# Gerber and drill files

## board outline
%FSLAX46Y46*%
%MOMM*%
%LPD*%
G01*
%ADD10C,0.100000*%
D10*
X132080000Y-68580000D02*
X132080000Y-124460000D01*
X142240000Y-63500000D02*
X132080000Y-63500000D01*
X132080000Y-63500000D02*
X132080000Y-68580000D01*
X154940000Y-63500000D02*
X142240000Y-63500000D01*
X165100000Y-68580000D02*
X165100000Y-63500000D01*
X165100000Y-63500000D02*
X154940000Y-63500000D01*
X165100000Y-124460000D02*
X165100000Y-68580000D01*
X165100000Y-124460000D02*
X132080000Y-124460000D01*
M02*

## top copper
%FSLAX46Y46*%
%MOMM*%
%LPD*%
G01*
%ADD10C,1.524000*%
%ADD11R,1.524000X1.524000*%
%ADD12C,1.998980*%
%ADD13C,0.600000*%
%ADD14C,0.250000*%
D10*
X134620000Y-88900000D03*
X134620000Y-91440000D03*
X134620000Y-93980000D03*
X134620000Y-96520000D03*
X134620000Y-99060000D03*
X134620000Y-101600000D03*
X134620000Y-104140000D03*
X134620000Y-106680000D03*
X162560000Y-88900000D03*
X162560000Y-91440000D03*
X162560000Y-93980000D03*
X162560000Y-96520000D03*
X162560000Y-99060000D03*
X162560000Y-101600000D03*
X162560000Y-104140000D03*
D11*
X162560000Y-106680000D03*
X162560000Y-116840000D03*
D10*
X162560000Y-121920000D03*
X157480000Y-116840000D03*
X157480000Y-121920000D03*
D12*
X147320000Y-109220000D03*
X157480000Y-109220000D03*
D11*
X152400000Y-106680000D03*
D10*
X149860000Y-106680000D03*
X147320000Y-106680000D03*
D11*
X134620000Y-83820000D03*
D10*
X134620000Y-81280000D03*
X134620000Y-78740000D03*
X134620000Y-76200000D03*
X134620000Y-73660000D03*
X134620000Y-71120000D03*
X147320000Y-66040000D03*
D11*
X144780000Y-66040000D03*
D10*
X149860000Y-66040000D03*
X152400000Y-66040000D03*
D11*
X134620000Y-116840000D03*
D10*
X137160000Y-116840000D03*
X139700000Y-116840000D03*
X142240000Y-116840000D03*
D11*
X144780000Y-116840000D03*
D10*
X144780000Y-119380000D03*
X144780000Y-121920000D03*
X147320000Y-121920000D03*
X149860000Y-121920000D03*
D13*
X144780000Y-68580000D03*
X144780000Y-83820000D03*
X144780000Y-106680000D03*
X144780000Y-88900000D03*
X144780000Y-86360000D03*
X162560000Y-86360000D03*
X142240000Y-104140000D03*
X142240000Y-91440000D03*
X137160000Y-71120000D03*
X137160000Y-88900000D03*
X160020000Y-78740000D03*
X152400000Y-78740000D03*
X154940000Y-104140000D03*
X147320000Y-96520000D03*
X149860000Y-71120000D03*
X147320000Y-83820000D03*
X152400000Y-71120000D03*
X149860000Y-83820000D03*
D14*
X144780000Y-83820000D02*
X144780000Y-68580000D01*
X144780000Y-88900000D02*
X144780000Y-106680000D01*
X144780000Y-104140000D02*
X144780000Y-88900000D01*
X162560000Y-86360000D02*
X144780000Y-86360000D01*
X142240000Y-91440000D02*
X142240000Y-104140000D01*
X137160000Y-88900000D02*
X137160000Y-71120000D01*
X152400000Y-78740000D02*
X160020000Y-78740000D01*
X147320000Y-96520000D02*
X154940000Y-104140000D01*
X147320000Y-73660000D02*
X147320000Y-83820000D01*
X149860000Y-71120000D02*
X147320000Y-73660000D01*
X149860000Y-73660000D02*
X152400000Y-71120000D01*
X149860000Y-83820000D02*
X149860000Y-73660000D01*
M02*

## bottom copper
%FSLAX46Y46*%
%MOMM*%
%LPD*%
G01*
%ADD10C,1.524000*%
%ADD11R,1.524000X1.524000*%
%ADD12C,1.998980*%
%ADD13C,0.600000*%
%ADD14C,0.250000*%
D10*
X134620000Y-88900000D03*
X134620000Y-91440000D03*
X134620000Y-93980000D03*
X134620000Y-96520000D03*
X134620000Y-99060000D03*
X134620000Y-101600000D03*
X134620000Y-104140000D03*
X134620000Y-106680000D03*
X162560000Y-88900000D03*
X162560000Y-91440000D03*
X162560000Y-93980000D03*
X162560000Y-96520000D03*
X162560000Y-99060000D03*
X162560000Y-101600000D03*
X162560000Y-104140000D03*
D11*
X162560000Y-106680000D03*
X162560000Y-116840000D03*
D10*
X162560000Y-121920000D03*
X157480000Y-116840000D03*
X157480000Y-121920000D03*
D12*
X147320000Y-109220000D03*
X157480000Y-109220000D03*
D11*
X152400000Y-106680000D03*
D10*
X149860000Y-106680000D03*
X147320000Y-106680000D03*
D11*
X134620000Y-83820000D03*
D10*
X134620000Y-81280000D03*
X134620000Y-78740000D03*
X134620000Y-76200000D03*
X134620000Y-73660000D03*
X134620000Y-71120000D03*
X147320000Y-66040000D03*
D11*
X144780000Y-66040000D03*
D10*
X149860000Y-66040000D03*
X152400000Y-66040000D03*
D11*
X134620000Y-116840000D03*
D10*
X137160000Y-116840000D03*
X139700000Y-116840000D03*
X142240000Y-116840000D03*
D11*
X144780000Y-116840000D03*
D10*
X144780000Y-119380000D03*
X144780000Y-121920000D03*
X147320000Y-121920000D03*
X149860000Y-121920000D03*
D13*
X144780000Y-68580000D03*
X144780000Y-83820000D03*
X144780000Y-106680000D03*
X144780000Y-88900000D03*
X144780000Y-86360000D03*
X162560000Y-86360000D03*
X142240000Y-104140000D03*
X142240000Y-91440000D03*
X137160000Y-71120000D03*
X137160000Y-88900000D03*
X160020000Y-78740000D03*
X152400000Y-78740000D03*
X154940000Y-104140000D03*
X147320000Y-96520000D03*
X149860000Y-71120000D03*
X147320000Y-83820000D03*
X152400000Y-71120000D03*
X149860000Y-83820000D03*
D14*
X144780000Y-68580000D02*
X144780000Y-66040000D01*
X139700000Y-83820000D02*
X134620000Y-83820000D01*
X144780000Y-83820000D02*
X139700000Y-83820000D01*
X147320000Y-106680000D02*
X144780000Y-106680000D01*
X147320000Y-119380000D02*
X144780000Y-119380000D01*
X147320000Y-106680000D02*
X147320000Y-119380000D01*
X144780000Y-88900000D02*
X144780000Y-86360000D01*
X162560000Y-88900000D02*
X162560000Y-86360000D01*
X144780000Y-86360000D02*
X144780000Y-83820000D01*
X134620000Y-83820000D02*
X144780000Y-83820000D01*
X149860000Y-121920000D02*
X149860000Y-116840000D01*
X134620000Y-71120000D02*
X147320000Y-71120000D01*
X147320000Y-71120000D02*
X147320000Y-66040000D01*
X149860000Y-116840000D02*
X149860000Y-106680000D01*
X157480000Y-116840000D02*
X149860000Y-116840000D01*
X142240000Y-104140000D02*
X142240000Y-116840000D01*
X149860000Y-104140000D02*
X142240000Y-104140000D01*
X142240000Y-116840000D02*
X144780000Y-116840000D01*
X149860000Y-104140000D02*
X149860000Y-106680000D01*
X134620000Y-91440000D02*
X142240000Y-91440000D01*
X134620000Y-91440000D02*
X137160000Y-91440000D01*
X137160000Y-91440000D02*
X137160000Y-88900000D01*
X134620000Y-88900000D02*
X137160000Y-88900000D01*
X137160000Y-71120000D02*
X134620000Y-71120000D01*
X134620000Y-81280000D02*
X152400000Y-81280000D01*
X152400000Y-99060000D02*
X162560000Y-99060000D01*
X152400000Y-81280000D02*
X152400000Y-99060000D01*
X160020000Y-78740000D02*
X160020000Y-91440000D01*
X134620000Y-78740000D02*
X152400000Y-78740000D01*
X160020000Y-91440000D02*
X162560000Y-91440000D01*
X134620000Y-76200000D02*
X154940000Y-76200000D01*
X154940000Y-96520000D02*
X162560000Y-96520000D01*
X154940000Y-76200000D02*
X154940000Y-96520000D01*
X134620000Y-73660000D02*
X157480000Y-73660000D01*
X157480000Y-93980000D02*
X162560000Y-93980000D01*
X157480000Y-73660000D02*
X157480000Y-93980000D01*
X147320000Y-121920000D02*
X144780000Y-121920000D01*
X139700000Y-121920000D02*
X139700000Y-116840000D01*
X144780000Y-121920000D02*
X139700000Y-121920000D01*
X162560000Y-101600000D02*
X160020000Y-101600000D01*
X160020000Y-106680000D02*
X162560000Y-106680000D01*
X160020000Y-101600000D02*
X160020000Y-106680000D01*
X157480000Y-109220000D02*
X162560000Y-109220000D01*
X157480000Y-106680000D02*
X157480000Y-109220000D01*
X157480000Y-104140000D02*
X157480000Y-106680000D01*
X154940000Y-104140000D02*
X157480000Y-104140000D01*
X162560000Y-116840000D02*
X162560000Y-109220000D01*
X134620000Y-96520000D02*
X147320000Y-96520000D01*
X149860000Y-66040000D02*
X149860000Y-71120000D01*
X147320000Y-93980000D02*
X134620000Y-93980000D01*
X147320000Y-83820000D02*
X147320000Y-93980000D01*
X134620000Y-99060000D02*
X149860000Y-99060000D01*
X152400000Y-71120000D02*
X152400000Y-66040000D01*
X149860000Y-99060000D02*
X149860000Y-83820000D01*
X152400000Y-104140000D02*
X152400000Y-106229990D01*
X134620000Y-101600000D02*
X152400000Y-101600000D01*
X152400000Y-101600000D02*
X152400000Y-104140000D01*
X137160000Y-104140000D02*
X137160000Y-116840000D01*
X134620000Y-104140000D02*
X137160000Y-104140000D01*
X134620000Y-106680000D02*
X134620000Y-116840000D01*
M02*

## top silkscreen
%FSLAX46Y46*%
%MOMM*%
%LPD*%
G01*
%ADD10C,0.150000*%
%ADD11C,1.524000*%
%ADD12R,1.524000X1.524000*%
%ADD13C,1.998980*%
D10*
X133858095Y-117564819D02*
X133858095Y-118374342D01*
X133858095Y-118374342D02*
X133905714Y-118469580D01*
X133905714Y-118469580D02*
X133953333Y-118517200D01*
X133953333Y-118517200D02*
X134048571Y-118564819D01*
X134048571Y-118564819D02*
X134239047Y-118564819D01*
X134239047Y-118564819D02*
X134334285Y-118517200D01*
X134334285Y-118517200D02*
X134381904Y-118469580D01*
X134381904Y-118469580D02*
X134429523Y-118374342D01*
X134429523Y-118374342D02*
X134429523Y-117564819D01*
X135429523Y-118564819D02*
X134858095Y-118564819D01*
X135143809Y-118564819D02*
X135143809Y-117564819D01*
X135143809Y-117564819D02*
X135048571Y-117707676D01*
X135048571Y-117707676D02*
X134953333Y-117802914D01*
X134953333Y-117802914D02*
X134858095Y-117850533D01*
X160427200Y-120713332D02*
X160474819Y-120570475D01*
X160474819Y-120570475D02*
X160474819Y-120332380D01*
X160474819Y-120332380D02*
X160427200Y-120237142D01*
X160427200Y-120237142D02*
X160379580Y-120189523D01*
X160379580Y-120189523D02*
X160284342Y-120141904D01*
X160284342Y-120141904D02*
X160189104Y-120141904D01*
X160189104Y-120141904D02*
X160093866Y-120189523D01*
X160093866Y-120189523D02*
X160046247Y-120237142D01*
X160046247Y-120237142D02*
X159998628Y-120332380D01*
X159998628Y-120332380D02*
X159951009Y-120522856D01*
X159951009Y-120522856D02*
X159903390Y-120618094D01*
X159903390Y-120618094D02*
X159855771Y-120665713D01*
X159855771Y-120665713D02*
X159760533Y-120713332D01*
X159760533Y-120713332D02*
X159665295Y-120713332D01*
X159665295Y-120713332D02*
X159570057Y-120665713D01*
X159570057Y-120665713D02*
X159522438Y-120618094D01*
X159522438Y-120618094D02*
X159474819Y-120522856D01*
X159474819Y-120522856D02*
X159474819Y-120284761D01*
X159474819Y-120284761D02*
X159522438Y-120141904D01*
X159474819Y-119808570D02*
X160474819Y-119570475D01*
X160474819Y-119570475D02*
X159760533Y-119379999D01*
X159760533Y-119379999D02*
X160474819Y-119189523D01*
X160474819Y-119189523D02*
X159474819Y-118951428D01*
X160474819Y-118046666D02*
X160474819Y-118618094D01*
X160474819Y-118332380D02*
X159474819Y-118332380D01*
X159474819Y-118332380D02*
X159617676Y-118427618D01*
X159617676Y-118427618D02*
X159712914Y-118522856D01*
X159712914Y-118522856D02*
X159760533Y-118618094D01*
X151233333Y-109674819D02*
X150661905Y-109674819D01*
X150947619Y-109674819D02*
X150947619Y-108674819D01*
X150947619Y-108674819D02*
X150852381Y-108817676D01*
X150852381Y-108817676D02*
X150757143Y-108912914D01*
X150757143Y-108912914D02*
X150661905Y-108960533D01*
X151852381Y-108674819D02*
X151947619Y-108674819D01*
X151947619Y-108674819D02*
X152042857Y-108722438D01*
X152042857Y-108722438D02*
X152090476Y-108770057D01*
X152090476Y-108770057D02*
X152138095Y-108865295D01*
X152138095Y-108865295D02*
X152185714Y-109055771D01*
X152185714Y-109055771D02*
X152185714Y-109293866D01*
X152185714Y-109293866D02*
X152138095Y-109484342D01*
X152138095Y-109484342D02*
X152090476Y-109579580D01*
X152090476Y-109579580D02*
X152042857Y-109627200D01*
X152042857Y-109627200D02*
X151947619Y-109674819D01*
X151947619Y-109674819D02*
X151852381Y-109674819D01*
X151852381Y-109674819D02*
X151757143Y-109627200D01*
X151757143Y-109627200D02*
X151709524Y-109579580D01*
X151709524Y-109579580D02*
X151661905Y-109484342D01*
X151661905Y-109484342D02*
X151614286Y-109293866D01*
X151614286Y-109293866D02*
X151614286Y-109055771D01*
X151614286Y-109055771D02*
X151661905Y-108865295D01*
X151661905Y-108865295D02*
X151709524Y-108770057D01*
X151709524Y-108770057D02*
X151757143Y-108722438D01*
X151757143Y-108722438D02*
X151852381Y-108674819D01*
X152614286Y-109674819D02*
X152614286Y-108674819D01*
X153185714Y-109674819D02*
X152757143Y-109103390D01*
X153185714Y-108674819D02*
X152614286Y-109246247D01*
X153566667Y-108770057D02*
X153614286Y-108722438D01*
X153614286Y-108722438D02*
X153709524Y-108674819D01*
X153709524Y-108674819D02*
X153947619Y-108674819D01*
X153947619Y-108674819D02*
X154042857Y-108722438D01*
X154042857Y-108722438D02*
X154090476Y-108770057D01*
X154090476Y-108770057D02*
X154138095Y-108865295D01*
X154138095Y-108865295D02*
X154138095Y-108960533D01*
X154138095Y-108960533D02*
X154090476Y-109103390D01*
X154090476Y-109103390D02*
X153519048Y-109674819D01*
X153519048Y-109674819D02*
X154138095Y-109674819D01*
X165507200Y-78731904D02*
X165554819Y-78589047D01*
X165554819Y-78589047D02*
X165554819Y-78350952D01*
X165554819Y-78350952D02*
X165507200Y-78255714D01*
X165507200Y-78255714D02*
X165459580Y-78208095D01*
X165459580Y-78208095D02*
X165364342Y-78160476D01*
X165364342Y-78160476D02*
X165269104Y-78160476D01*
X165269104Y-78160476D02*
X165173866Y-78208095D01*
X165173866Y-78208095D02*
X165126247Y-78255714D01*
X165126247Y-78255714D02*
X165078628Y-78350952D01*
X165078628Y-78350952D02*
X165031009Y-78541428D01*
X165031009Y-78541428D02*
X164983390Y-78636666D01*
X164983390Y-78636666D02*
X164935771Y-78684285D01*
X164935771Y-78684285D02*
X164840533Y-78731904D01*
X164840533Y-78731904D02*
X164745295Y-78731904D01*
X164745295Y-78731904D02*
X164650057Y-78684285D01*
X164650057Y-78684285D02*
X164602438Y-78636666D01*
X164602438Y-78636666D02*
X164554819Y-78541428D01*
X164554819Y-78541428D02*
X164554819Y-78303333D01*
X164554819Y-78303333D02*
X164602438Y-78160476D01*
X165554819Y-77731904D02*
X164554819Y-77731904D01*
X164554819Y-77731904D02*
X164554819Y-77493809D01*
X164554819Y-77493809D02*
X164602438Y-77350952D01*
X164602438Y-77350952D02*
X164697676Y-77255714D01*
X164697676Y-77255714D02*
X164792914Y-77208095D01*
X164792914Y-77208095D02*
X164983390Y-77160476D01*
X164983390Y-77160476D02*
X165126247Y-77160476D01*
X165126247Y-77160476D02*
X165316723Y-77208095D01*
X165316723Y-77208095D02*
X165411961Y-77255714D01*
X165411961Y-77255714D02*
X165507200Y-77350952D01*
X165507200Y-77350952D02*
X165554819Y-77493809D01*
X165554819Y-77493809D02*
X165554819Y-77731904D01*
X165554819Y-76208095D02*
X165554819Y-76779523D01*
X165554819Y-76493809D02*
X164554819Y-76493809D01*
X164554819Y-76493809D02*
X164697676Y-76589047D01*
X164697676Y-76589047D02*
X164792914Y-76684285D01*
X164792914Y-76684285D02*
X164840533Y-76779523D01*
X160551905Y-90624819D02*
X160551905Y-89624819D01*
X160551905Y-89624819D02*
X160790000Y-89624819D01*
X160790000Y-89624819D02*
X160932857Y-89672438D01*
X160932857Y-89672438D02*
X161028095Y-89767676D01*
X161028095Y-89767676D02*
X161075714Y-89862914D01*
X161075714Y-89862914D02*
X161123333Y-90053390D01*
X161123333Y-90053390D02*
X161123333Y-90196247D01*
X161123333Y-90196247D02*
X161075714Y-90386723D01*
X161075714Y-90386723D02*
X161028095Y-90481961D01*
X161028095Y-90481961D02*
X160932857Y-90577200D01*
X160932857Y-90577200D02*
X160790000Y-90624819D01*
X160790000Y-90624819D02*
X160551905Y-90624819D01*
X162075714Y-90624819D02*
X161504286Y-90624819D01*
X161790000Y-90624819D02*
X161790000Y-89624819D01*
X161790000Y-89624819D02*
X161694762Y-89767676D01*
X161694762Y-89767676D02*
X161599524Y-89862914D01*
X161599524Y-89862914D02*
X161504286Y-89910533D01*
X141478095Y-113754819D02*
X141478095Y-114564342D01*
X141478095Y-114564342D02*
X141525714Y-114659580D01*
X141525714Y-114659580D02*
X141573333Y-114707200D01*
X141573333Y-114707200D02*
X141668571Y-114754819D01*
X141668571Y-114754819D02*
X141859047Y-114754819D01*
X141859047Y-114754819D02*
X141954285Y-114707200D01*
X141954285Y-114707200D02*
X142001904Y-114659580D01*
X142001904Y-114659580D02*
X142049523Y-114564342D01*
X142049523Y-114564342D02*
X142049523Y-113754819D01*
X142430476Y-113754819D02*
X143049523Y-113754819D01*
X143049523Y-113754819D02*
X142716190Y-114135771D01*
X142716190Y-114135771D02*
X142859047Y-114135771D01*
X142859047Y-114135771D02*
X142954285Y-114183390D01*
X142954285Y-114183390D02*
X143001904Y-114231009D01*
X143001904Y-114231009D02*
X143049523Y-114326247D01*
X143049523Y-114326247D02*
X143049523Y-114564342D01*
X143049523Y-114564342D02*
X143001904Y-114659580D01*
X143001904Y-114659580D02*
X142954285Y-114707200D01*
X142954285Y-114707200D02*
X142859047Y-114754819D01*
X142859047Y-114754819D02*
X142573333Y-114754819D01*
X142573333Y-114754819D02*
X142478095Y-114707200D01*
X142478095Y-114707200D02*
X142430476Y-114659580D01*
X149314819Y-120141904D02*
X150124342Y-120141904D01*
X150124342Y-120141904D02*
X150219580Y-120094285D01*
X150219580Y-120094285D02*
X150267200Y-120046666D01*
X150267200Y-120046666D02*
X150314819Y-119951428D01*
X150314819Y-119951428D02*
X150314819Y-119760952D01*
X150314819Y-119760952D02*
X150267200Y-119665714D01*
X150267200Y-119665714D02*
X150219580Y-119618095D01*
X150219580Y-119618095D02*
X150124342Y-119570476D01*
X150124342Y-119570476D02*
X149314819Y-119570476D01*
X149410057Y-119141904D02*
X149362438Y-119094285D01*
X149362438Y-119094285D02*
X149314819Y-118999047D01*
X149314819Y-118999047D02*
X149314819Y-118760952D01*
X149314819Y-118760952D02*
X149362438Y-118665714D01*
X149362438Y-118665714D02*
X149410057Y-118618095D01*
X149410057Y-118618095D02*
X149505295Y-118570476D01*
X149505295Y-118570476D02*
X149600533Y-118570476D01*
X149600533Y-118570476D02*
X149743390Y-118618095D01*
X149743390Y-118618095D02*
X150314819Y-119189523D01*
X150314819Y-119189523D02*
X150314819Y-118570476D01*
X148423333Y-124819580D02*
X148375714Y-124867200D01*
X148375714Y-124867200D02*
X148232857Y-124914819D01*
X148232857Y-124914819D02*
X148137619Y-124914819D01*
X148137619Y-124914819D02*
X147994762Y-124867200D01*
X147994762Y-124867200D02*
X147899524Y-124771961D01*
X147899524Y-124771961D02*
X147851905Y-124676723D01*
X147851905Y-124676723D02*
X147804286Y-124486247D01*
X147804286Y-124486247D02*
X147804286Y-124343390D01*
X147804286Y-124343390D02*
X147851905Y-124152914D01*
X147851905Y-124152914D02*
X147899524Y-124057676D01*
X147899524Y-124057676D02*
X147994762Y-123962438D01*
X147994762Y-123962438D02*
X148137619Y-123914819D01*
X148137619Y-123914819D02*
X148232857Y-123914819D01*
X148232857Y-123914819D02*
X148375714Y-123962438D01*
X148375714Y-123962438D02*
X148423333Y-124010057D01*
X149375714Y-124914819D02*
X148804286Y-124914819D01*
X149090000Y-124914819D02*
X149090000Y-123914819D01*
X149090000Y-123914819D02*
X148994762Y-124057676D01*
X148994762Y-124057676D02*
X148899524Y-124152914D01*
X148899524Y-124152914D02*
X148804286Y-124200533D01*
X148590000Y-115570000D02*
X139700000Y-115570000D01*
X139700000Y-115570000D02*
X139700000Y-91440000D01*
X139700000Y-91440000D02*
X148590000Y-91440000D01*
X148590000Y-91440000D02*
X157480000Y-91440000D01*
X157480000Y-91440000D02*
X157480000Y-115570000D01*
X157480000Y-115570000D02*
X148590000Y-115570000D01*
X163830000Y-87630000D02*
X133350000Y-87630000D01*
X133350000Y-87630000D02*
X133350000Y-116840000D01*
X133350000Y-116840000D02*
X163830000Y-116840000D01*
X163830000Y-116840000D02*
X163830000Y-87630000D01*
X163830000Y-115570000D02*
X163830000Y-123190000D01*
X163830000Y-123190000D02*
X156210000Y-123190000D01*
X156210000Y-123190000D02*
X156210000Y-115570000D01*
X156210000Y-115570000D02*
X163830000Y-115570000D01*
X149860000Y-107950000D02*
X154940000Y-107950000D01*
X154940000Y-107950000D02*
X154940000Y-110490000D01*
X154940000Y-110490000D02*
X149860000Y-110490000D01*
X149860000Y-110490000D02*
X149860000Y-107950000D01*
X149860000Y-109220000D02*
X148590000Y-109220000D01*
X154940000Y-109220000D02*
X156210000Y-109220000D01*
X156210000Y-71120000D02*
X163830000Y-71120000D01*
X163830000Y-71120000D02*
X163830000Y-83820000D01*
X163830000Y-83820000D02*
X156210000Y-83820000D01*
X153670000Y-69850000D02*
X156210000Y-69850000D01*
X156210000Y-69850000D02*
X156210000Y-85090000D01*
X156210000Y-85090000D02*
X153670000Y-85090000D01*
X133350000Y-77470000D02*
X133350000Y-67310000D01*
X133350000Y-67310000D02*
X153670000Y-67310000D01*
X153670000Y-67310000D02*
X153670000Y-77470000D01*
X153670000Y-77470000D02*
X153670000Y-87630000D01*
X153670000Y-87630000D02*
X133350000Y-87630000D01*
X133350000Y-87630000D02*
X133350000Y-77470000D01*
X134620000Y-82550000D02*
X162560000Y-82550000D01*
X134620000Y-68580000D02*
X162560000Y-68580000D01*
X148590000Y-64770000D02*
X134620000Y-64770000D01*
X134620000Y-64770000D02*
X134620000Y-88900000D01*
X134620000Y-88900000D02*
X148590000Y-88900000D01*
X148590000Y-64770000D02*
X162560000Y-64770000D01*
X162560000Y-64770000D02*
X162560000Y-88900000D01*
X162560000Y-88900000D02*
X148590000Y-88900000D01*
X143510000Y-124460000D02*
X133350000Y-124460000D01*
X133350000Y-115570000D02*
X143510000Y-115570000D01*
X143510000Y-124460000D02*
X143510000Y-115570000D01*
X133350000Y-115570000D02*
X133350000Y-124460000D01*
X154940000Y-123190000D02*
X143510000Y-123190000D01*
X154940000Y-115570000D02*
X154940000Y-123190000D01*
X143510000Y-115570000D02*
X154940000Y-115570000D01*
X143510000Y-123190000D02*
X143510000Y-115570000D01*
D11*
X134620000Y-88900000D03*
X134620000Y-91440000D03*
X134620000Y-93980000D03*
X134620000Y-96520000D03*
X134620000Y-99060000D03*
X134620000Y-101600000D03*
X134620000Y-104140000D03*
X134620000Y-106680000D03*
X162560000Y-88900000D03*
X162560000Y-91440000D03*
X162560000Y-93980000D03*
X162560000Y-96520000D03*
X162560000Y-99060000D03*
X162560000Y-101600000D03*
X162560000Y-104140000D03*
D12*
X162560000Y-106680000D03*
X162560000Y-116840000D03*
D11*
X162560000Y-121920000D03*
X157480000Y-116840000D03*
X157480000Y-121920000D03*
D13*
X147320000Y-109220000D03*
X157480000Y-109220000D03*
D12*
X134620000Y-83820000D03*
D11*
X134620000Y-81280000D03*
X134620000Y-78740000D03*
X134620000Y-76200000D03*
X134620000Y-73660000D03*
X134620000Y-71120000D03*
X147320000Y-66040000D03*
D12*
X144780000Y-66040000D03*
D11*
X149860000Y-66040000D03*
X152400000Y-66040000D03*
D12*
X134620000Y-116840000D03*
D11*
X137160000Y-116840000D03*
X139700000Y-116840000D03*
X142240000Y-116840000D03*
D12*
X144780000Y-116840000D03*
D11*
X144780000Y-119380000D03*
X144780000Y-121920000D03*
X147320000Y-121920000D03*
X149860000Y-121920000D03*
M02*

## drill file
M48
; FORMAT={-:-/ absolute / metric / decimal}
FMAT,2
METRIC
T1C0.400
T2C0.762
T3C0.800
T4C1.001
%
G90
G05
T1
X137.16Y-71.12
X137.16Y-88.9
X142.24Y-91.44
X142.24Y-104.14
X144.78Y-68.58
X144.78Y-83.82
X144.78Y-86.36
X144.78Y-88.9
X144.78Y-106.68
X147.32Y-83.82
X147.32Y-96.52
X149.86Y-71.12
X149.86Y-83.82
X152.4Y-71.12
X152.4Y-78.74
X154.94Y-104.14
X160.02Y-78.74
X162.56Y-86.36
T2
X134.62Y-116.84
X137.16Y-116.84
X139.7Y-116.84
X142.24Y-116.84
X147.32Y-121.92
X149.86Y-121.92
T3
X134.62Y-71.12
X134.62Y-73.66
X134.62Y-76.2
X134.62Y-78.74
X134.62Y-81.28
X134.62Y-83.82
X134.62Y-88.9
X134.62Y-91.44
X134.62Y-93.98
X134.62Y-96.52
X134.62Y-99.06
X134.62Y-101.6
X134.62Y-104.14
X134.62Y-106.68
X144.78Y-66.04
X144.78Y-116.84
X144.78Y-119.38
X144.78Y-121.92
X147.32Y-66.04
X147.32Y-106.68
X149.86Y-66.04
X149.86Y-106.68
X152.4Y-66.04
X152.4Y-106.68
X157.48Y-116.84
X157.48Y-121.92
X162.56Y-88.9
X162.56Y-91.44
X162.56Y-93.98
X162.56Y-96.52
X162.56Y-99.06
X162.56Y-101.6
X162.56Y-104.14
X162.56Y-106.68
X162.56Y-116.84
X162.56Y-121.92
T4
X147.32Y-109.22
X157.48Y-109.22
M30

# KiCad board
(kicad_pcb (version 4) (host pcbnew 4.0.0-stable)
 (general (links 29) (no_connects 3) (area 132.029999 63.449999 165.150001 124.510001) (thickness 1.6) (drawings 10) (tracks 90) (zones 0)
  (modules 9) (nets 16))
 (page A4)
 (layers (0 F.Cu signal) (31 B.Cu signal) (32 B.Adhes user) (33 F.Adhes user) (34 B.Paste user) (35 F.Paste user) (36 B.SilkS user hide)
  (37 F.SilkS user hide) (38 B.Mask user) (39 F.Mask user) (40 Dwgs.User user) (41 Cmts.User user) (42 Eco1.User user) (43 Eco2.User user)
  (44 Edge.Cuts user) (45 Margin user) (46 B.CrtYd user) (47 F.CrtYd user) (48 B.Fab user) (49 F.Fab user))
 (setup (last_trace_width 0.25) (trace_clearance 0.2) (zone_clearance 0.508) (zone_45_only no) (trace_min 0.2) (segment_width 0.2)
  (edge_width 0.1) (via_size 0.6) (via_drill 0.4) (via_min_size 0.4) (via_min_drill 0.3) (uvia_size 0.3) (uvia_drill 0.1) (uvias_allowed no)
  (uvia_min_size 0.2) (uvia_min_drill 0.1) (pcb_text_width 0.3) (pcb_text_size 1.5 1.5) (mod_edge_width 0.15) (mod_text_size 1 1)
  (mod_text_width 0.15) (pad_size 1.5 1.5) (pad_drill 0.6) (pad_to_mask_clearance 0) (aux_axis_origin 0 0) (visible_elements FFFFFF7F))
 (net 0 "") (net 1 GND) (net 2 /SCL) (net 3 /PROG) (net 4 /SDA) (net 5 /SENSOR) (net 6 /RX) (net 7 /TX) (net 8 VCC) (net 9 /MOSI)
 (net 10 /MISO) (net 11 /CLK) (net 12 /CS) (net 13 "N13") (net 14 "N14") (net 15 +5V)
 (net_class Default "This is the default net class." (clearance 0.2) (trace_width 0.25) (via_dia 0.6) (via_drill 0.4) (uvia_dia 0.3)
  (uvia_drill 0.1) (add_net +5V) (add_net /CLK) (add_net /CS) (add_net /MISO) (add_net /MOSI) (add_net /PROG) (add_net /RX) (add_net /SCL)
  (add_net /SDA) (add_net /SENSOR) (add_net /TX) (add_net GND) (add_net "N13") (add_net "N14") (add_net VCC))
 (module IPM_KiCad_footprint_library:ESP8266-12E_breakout (layer F.Cu) (at 162.56 106.68 180)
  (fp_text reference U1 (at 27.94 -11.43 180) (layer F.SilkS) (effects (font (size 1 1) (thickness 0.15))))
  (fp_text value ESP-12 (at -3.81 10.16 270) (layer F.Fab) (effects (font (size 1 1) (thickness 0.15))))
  (fp_line (start 13.97 -8.89) (end 22.86 -8.89) (layer F.SilkS) (width 0.15))
  (fp_line (start 22.86 -8.89) (end 22.86 15.24) (layer F.SilkS) (width 0.15))
  (fp_line (start 22.86 15.24) (end 13.97 15.24) (layer F.SilkS) (width 0.15))
  (fp_line (start 13.97 15.24) (end 5.08 15.24) (layer F.SilkS) (width 0.15))
  (fp_line (start 5.08 15.24) (end 5.08 -8.89) (layer F.SilkS) (width 0.15))
  (fp_line (start 5.08 -8.89) (end 13.97 -8.89) (layer F.SilkS) (width 0.15))
  (fp_line (start -1.27 19.05) (end 29.21 19.05) (layer F.SilkS) (width 0.15))
  (fp_line (start 29.21 19.05) (end 29.21 -10.16) (layer F.SilkS) (width 0.15))
  (fp_line (start 29.21 -10.16) (end -1.27 -10.16) (layer F.SilkS) (width 0.15))
  (fp_line (start -1.27 -10.16) (end -1.27 19.05) (layer F.SilkS) (width 0.15))
  (pad 9 thru_hole circle (at 27.94 17.78 180) (size 1.524 1.524) (drill 0.8) (layers *.Cu *.Mask F.SilkS) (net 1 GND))
  (pad 10 thru_hole circle (at 27.94 15.24 180) (size 1.524 1.524) (drill 0.8) (layers *.Cu *.Mask F.SilkS) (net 1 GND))
  (pad 11 thru_hole circle (at 27.94 12.7 180) (size 1.524 1.524) (drill 0.8) (layers *.Cu *.Mask F.SilkS) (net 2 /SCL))
  (pad 12 thru_hole circle (at 27.94 10.16 180) (size 1.524 1.524) (drill 0.8) (layers *.Cu *.Mask F.SilkS) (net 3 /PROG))
  (pad 13 thru_hole circle (at 27.94 7.62 180) (size 1.524 1.524) (drill 0.8) (layers *.Cu *.Mask F.SilkS) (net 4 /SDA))
  (pad 14 thru_hole circle (at 27.94 5.08 180) (size 1.524 1.524) (drill 0.8) (layers *.Cu *.Mask F.SilkS) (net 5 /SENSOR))
  (pad 15 thru_hole circle (at 27.94 2.54 180) (size 1.524 1.524) (drill 0.8) (layers *.Cu *.Mask F.SilkS) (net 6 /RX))
  (pad 16 thru_hole circle (at 27.94 0 180) (size 1.524 1.524) (drill 0.8) (layers *.Cu *.Mask F.SilkS) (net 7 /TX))
  (pad 8 thru_hole circle (at 0 17.78 180) (size 1.524 1.524) (drill 0.8) (layers *.Cu *.Mask F.SilkS) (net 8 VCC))
  (pad 7 thru_hole circle (at 0 15.24 180) (size 1.524 1.524) (drill 0.8) (layers *.Cu *.Mask F.SilkS) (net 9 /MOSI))
  (pad 6 thru_hole circle (at 0 12.7 180) (size 1.524 1.524) (drill 0.8) (layers *.Cu *.Mask F.SilkS) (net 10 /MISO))
  (pad 5 thru_hole circle (at 0 10.16 180) (size 1.524 1.524) (drill 0.8) (layers *.Cu *.Mask F.SilkS) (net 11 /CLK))
  (pad 4 thru_hole circle (at 0 7.62 180) (size 1.524 1.524) (drill 0.8) (layers *.Cu *.Mask F.SilkS) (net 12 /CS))
  (pad 3 thru_hole circle (at 0 5.08 180) (size 1.524 1.524) (drill 0.8) (layers *.Cu *.Mask F.SilkS) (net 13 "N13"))
  (pad 2 thru_hole circle (at 0 2.54 180) (size 1.524 1.524) (drill 0.8) (layers *.Cu *.Mask F.SilkS) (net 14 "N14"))
  (pad 1 thru_hole rect (at 0 0 180) (size 1.524 1.524) (drill 0.8) (layers *.Cu *.Mask F.SilkS) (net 13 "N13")))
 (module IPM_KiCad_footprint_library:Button (layer F.Cu) (at 162.56 116.84 270)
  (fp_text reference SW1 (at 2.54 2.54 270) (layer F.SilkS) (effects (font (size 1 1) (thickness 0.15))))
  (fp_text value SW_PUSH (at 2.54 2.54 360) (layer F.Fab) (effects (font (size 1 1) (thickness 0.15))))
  (fp_line (start -1.27 -1.27) (end 6.35 -1.27) (layer F.SilkS) (width 0.15))
  (fp_line (start 6.35 -1.27) (end 6.35 6.35) (layer F.SilkS) (width 0.15))
  (fp_line (start 6.35 6.35) (end -1.27 6.35) (layer F.SilkS) (width 0.15))
  (fp_line (start -1.27 6.35) (end -1.27 -1.27) (layer F.SilkS) (width 0.15))
  (pad 1 thru_hole rect (at 0 0 270) (size 1.524 1.524) (drill 0.8) (layers *.Cu *.Mask F.SilkS) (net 3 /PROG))
  (pad 1 thru_hole circle (at 5.08 0 270) (size 1.524 1.524) (drill 0.8) (layers *.Cu *.Mask F.SilkS) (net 3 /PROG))
  (pad 2 thru_hole circle (at 0 5.08 270) (size 1.524 1.524) (drill 0.8) (layers *.Cu *.Mask F.SilkS) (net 1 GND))
  (pad 2 thru_hole circle (at 5.08 5.08 270) (size 1.524 1.524) (drill 0.8) (layers *.Cu *.Mask F.SilkS) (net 1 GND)))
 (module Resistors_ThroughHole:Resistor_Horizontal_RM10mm (layer F.Cu) (at 152.4 109.22)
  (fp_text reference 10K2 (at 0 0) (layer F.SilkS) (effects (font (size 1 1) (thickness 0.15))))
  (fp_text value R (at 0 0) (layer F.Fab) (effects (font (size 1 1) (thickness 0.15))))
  (fp_line (start -2.54 -1.27) (end 2.54 -1.27) (layer F.SilkS) (width 0.15))
  (fp_line (start 2.54 -1.27) (end 2.54 1.27) (layer F.SilkS) (width 0.15))
  (fp_line (start 2.54 1.27) (end -2.54 1.27) (layer F.SilkS) (width 0.15))
  (fp_line (start -2.54 1.27) (end -2.54 -1.27) (layer F.SilkS) (width 0.15))
  (fp_line (start -2.54 0) (end -3.81 0) (layer F.SilkS) (width 0.15))
  (fp_line (start 2.54 0) (end 3.81 0) (layer F.SilkS) (width 0.15))
  (pad 1 thru_hole circle (at -5.08 0) (size 1.99898 1.99898) (drill 1.00076) (layers *.Cu *.SilkS *.Mask) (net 8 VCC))
  (pad 2 thru_hole circle (at 5.08 0) (size 1.99898 1.99898) (drill 1.00076) (layers *.Cu *.SilkS *.Mask) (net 3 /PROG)))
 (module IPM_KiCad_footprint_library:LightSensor (layer B.Cu) (at 152.4 106.68 180)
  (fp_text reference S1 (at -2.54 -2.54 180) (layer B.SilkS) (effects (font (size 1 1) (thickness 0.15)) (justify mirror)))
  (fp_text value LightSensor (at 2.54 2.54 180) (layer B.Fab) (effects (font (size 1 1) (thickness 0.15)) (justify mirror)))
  (pad 1 thru_hole rect (at 0 0 180) (size 1.524 1.524) (drill 0.8) (layers *.Cu *.Mask B.SilkS) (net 5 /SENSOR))
  (pad 2 thru_hole circle (at 2.54 0 180) (size 1.524 1.524) (drill 0.8) (layers *.Cu *.Mask B.SilkS) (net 1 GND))
  (pad 3 thru_hole circle (at 5.08 0 180) (size 1.524 1.524) (drill 0.8) (layers *.Cu *.Mask B.SilkS) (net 8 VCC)))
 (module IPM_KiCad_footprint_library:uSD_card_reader (layer F.Cu) (at 134.62 83.82 90)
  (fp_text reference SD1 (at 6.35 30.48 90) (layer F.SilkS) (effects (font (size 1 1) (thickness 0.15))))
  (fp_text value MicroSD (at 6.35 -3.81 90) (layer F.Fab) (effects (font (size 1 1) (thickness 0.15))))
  (fp_line (start 12.7 21.59) (end 12.7 29.21) (layer F.SilkS) (width 0.15))
  (fp_line (start 12.7 29.21) (end 0 29.21) (layer F.SilkS) (width 0.15))
  (fp_line (start 0 29.21) (end 0 21.59) (layer F.SilkS) (width 0.15))
  (fp_line (start 13.97 19.05) (end 13.97 21.59) (layer F.SilkS) (width 0.15))
  (fp_line (start 13.97 21.59) (end -1.27 21.59) (layer F.SilkS) (width 0.15))
  (fp_line (start -1.27 21.59) (end -1.27 19.05) (layer F.SilkS) (width 0.15))
  (fp_line (start 6.35 -1.27) (end 16.51 -1.27) (layer F.SilkS) (width 0.15))
  (fp_line (start 16.51 -1.27) (end 16.51 19.05) (layer F.SilkS) (width 0.15))
  (fp_line (start 16.51 19.05) (end 6.35 19.05) (layer F.SilkS) (width 0.15))
  (fp_line (start 6.35 19.05) (end -3.81 19.05) (layer F.SilkS) (width 0.15))
  (fp_line (start -3.81 19.05) (end -3.81 -1.27) (layer F.SilkS) (width 0.15))
  (fp_line (start -3.81 -1.27) (end 6.35 -1.27) (layer F.SilkS) (width 0.15))
  (pad 1 thru_hole rect (at 0 0 90) (size 1.524 1.524) (drill 0.8) (layers *.Cu *.Mask F.SilkS) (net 8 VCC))
  (pad 2 thru_hole circle (at 2.54 0 90) (size 1.524 1.524) (drill 0.8) (layers *.Cu *.Mask F.SilkS) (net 12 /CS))
  (pad 3 thru_hole circle (at 5.08 0 90) (size 1.524 1.524) (drill 0.8) (layers *.Cu *.Mask F.SilkS) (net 9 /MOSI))
  (pad 4 thru_hole circle (at 7.62 0 90) (size 1.524 1.524) (drill 0.8) (layers *.Cu *.Mask F.SilkS) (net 11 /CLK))
  (pad 5 thru_hole circle (at 10.16 0 90) (size 1.524 1.524) (drill 0.8) (layers *.Cu *.Mask F.SilkS) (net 10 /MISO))
  (pad 6 thru_hole circle (at 12.7 0 90) (size 1.524 1.524) (drill 0.8) (layers *.Cu *.Mask F.SilkS) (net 1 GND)))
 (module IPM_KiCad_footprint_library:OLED (layer F.Cu) (at 144.78 66.04)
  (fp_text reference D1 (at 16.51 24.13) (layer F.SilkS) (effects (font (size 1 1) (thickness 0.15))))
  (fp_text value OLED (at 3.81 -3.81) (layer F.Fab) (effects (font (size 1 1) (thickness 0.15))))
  (fp_line (start -10.16 16.51) (end 17.78 16.51) (layer F.SilkS) (width 0.15))
  (fp_line (start -10.16 2.54) (end 17.78 2.54) (layer F.SilkS) (width 0.15))
  (fp_line (start 3.81 -1.27) (end -10.16 -1.27) (layer F.SilkS) (width 0.15))
  (fp_line (start -10.16 -1.27) (end -10.16 22.86) (layer F.SilkS) (width 0.15))
  (fp_line (start -10.16 22.86) (end 3.81 22.86) (layer F.SilkS) (width 0.15))
  (fp_line (start 3.81 -1.27) (end 17.78 -1.27) (layer F.SilkS) (width 0.15))
  (fp_line (start 17.78 -1.27) (end 17.78 22.86) (layer F.SilkS) (width 0.15))
  (fp_line (start 17.78 22.86) (end 3.81 22.86) (layer F.SilkS) (width 0.15))
  (pad 2 thru_hole circle (at 2.54 0) (size 1.524 1.524) (drill 0.8) (layers *.Cu *.Mask F.SilkS) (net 1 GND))
  (pad 1 thru_hole rect (at 0 0) (size 1.524 1.524) (drill 0.8) (layers *.Cu *.Mask F.SilkS) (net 8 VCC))
  (pad 3 thru_hole circle (at 5.08 0) (size 1.524 1.524) (drill 0.8) (layers *.Cu *.Mask F.SilkS) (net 2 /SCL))
  (pad 4 thru_hole circle (at 7.62 0) (size 1.524 1.524) (drill 0.8) (layers *.Cu *.Mask F.SilkS) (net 4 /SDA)))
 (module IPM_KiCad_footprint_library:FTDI (layer F.Cu) (at 134.62 116.84)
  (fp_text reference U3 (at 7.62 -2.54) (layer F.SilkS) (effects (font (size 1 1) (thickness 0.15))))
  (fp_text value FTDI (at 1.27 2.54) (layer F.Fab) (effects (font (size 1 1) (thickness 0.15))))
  (fp_line (start 8.89 7.62) (end -1.27 7.62) (layer F.SilkS) (width 0.15))
  (fp_line (start -1.27 -1.27) (end 8.89 -1.27) (layer F.SilkS) (width 0.15))
  (fp_line (start 8.89 7.62) (end 8.89 -1.27) (layer F.SilkS) (width 0.15))
  (fp_line (start -1.27 -1.27) (end -1.27 7.62) (layer F.SilkS) (width 0.15))
  (pad 1 thru_hole rect (at 0 0) (size 1.524 1.524) (drill 0.762) (layers *.Cu *.Mask F.SilkS) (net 7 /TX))
  (pad 2 thru_hole circle (at 2.54 0) (size 1.524 1.524) (drill 0.762) (layers *.Cu *.Mask F.SilkS) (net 6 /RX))
  (pad 3 thru_hole circle (at 5.08 0) (size 1.524 1.524) (drill 0.762) (layers *.Cu *.Mask F.SilkS) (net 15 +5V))
  (pad 4 thru_hole circle (at 7.62 0) (size 1.524 1.524) (drill 0.762) (layers *.Cu *.Mask F.SilkS) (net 1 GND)))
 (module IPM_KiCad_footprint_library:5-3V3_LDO (layer F.Cu) (at 144.78 116.84 90)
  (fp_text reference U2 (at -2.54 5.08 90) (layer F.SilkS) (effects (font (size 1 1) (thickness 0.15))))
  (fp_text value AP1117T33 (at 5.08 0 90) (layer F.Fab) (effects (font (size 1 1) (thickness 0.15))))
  (fp_line (start -6.35 10.16) (end -6.35 -1.27) (layer F.SilkS) (width 0.15))
  (fp_line (start 1.27 10.16) (end -6.35 10.16) (layer F.SilkS) (width 0.15))
  (fp_line (start 1.27 -1.27) (end 1.27 10.16) (layer F.SilkS) (width 0.15))
  (fp_line (start -6.35 -1.27) (end 1.27 -1.27) (layer F.SilkS) (width 0.15))
  (pad 1 thru_hole rect (at 0 0 90) (size 1.524 1.524) (drill 0.8) (layers *.Cu *.Mask F.SilkS) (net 1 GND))
  (pad 2 thru_hole circle (at -2.54 0 90) (size 1.524 1.524) (drill 0.8) (layers *.Cu *.Mask F.SilkS) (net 8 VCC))
  (pad 3 thru_hole circle (at -5.08 0 90) (size 1.524 1.524) (drill 0.8) (layers *.Cu *.Mask F.SilkS) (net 15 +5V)))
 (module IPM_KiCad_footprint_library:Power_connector (layer F.Cu) (at 148.59 121.92)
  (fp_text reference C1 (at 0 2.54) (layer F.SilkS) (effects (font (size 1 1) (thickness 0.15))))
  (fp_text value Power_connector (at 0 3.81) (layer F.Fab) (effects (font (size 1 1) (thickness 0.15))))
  (pad 1 thru_hole circle (at -1.27 0) (size 1.524 1.524) (drill 0.762) (layers *.Cu *.Mask F.SilkS) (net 15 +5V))
  (pad 2 thru_hole circle (at 1.27 0) (size 1.524 1.524) (drill 0.762) (layers *.Cu *.Mask F.SilkS) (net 1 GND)))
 (gr_line (start 132.08 68.58) (end 132.08 124.46) (angle 90) (layer Edge.Cuts) (width 0.1))
 (gr_line (start 142.24 63.5) (end 132.08 63.5) (angle 90) (layer Edge.Cuts) (width 0.1))
 (gr_line (start 132.08 63.5) (end 132.08 68.58) (angle 90) (layer Edge.Cuts) (width 0.1))
 (gr_line (start 154.94 63.5) (end 142.24 63.5) (angle 90) (layer Edge.Cuts) (width 0.1))
 (gr_line (start 165.1 68.58) (end 165.1 63.5) (angle 90) (layer Edge.Cuts) (width 0.1))
 (gr_line (start 165.1 63.5) (end 154.94 63.5) (angle 90) (layer Edge.Cuts) (width 0.1))
 (gr_line (start 165.1 124.46) (end 165.1 68.58) (angle 90) (layer Edge.Cuts) (width 0.1))
 (gr_line (start 165.1 124.46) (end 132.08 124.46) (angle 90) (layer Edge.Cuts) (width 0.1))
 (segment (start 144.78 68.58) (end 144.78 66.04) (width 0.25) (layer B.Cu) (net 8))
 (via (at 144.78 68.58) (size 0.6) (drill 0.4) (layers F.Cu B.Cu) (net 8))
 (segment (start 144.78 83.82) (end 144.78 68.58) (width 0.25) (layer F.Cu) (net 8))
 (segment (start 139.7 83.82) (end 134.62 83.82) (width 0.25) (layer B.Cu) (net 8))
 (segment (start 144.78 83.82) (end 139.7 83.82) (width 0.25) (layer B.Cu) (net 8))
 (via (at 144.78 83.82) (size 0.6) (drill 0.4) (layers F.Cu B.Cu) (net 8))
 (segment (start 144.78 88.9) (end 144.78 106.68) (width 0.25) (layer F.Cu) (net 8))
 (via (at 144.78 106.68) (size 0.6) (drill 0.4) (layers F.Cu B.Cu) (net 8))
 (segment (start 147.32 106.68) (end 144.78 106.68) (width 0.25) (layer B.Cu) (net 8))
 (segment (start 147.32 119.38) (end 144.78 119.38) (width 0.25) (layer B.Cu) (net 8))
 (segment (start 147.32 106.68) (end 147.32 119.38) (width 0.25) (layer B.Cu) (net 8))
 (segment (start 144.78 104.14) (end 144.78 88.9) (width 0.25) (layer F.Cu) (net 8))
 (segment (start 144.78 88.9) (end 144.78 86.36) (width 0.25) (layer B.Cu) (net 8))
 (via (at 144.78 88.9) (size 0.6) (drill 0.4) (layers F.Cu B.Cu) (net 8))
 (segment (start 162.56 88.9) (end 162.56 86.36) (width 0.25) (layer B.Cu) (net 8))
 (segment (start 144.78 86.36) (end 144.78 83.82) (width 0.25) (layer B.Cu) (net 8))
 (via (at 144.78 86.36) (size 0.6) (drill 0.4) (layers F.Cu B.Cu) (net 8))
 (segment (start 162.56 86.36) (end 144.78 86.36) (width 0.25) (layer F.Cu) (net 8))
 (via (at 162.56 86.36) (size 0.6) (drill 0.4) (layers F.Cu B.Cu) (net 8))
 (segment (start 134.62 83.82) (end 144.78 83.82) (width 0.25) (layer B.Cu) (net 8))
 (segment (start 149.86 121.92) (end 149.86 116.84) (width 0.25) (layer B.Cu) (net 1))
 (segment (start 134.62 71.12) (end 147.32 71.12) (width 0.25) (layer B.Cu) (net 1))
 (segment (start 147.32 71.12) (end 147.32 66.04) (width 0.25) (layer B.Cu) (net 1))
 (segment (start 149.86 116.84) (end 149.86 106.68) (width 0.25) (layer B.Cu) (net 1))
 (segment (start 157.48 116.84) (end 149.86 116.84) (width 0.25) (layer B.Cu) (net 1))
 (via (at 142.24 104.14) (size 0.6) (drill 0.4) (layers F.Cu B.Cu) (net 1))
 (segment (start 142.24 104.14) (end 142.24 116.84) (width 0.25) (layer B.Cu) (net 1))
 (segment (start 149.86 104.14) (end 142.24 104.14) (width 0.25) (layer B.Cu) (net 1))
 (segment (start 142.24 116.84) (end 144.78 116.84) (width 0.25) (layer B.Cu) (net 1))
 (segment (start 149.86 104.14) (end 149.86 106.68) (width 0.25) (layer B.Cu) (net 1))
 (segment (start 134.62 91.44) (end 142.24 91.44) (width 0.25) (layer B.Cu) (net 1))
 (segment (start 142.24 91.44) (end 142.24 104.14) (width 0.25) (layer F.Cu) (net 1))
 (via (at 142.24 91.44) (size 0.6) (drill 0.4) (layers F.Cu B.Cu) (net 1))
 (segment (start 134.62 91.44) (end 137.16 91.44) (width 0.25) (layer B.Cu) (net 1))
 (segment (start 137.16 91.44) (end 137.16 88.9) (width 0.25) (layer B.Cu) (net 1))
 (segment (start 134.62 88.9) (end 137.16 88.9) (width 0.25) (layer B.Cu) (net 1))
 (segment (start 137.16 71.12) (end 134.62 71.12) (width 0.25) (layer B.Cu) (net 1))
 (via (at 137.16 71.12) (size 0.6) (drill 0.4) (layers F.Cu B.Cu) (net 1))
 (segment (start 137.16 88.9) (end 137.16 71.12) (width 0.25) (layer F.Cu) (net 1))
 (via (at 137.16 88.9) (size 0.6) (drill 0.4) (layers F.Cu B.Cu) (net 1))
 (segment (start 134.62 81.28) (end 152.4 81.28) (width 0.25) (layer B.Cu) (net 12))
 (segment (start 152.4 99.06) (end 162.56 99.06) (width 0.25) (layer B.Cu) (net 12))
 (segment (start 152.4 81.28) (end 152.4 99.06) (width 0.25) (layer B.Cu) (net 12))
 (segment (start 152.4 78.74) (end 160.02 78.74) (width 0.25) (layer F.Cu) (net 9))
 (segment (start 160.02 78.74) (end 160.02 91.44) (width 0.25) (layer B.Cu) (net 9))
 (via (at 160.02 78.74) (size 0.6) (drill 0.4) (layers F.Cu B.Cu) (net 9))
 (segment (start 134.62 78.74) (end 152.4 78.74) (width 0.25) (layer B.Cu) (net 9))
 (segment (start 160.02 91.44) (end 162.56 91.44) (width 0.25) (layer B.Cu) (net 9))
 (via (at 152.4 78.74) (size 0.6) (drill 0.4) (layers F.Cu B.Cu) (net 9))
 (segment (start 134.62 76.2) (end 154.94 76.2) (width 0.25) (layer B.Cu) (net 11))
 (segment (start 154.94 96.52) (end 162.56 96.52) (width 0.25) (layer B.Cu) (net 11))
 (segment (start 154.94 76.2) (end 154.94 96.52) (width 0.25) (layer B.Cu) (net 11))
 (segment (start 134.62 73.66) (end 157.48 73.66) (width 0.25) (layer B.Cu) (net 10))
 (segment (start 157.48 93.98) (end 162.56 93.98) (width 0.25) (layer B.Cu) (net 10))
 (segment (start 157.48 73.66) (end 157.48 93.98) (width 0.25) (layer B.Cu) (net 10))
 (segment (start 147.32 121.92) (end 144.78 121.92) (width 0.25) (layer B.Cu) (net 15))
 (segment (start 139.7 121.92) (end 139.7 116.84) (width 0.25) (layer B.Cu) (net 15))
 (segment (start 144.78 121.92) (end 139.7 121.92) (width 0.25) (layer B.Cu) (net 15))
 (segment (start 162.56 101.6) (end 160.02 101.6) (width 0.25) (layer B.Cu) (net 13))
 (segment (start 160.02 106.68) (end 162.56 106.68) (width 0.25) (layer B.Cu) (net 13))
 (segment (start 160.02 101.6) (end 160.02 106.68) (width 0.25) (layer B.Cu) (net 13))
 (segment (start 157.48 109.22) (end 162.56 109.22) (width 0.25) (layer B.Cu) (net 3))
 (segment (start 157.48 106.68) (end 157.48 109.22) (width 0.25) (layer B.Cu) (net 3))
 (segment (start 157.48 104.14) (end 157.48 106.68) (width 0.25) (layer B.Cu) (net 3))
 (segment (start 154.94 104.14) (end 157.48 104.14) (width 0.25) (layer B.Cu) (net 3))
 (segment (start 162.56 116.84) (end 162.56 109.22) (width 0.25) (layer B.Cu) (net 3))
 (segment (start 134.62 96.52) (end 147.32 96.52) (width 0.25) (layer B.Cu) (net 3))
 (via (at 154.94 104.14) (size 0.6) (drill 0.4) (layers F.Cu B.Cu) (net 3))
 (segment (start 147.32 96.52) (end 154.94 104.14) (width 0.25) (layer F.Cu) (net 3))
 (via (at 147.32 96.52) (size 0.6) (drill 0.4) (layers F.Cu B.Cu) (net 3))
 (segment (start 149.86 66.04) (end 149.86 71.12) (width 0.25) (layer B.Cu) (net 2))
 (segment (start 147.32 73.66) (end 147.32 83.82) (width 0.25) (layer F.Cu) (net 2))
 (segment (start 149.86 71.12) (end 147.32 73.66) (width 0.25) (layer F.Cu) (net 2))
 (via (at 149.86 71.12) (size 0.6) (drill 0.4) (layers F.Cu B.Cu) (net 2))
 (segment (start 147.32 93.98) (end 134.62 93.98) (width 0.25) (layer B.Cu) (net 2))
 (segment (start 147.32 83.82) (end 147.32 93.98) (width 0.25) (layer B.Cu) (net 2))
 (via (at 147.32 83.82) (size 0.6) (drill 0.4) (layers F.Cu B.Cu) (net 2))
 (segment (start 149.86 73.66) (end 152.4 71.12) (width 0.25) (layer F.Cu) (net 4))
 (segment (start 149.86 83.82) (end 149.86 73.66) (width 0.25) (layer F.Cu) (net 4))
 (via (at 152.4 71.12) (size 0.6) (drill 0.4) (layers F.Cu B.Cu) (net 4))
 (segment (start 134.62 99.06) (end 149.86 99.06) (width 0.25) (layer B.Cu) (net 4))
 (segment (start 152.4 71.12) (end 152.4 66.04) (width 0.25) (layer B.Cu) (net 4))
 (via (at 149.86 83.82) (size 0.6) (drill 0.4) (layers F.Cu B.Cu) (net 4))
 (segment (start 149.86 99.06) (end 149.86 83.82) (width 0.25) (layer B.Cu) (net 4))
 (segment (start 152.4 104.14) (end 152.4 106.22999) (width 0.25) (layer B.Cu) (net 5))
 (segment (start 134.62 101.6) (end 152.4 101.6) (width 0.25) (layer B.Cu) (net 5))
 (segment (start 152.4 101.6) (end 152.4 104.14) (width 0.25) (layer B.Cu) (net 5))
 (segment (start 137.16 104.14) (end 137.16 116.84) (width 0.25) (layer B.Cu) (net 6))
 (segment (start 134.62 104.14) (end 137.16 104.14) (width 0.25) (layer B.Cu) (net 6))
 (segment (start 134.62 106.68) (end 134.62 116.84) (width 0.25) (layer B.Cu) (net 7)))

